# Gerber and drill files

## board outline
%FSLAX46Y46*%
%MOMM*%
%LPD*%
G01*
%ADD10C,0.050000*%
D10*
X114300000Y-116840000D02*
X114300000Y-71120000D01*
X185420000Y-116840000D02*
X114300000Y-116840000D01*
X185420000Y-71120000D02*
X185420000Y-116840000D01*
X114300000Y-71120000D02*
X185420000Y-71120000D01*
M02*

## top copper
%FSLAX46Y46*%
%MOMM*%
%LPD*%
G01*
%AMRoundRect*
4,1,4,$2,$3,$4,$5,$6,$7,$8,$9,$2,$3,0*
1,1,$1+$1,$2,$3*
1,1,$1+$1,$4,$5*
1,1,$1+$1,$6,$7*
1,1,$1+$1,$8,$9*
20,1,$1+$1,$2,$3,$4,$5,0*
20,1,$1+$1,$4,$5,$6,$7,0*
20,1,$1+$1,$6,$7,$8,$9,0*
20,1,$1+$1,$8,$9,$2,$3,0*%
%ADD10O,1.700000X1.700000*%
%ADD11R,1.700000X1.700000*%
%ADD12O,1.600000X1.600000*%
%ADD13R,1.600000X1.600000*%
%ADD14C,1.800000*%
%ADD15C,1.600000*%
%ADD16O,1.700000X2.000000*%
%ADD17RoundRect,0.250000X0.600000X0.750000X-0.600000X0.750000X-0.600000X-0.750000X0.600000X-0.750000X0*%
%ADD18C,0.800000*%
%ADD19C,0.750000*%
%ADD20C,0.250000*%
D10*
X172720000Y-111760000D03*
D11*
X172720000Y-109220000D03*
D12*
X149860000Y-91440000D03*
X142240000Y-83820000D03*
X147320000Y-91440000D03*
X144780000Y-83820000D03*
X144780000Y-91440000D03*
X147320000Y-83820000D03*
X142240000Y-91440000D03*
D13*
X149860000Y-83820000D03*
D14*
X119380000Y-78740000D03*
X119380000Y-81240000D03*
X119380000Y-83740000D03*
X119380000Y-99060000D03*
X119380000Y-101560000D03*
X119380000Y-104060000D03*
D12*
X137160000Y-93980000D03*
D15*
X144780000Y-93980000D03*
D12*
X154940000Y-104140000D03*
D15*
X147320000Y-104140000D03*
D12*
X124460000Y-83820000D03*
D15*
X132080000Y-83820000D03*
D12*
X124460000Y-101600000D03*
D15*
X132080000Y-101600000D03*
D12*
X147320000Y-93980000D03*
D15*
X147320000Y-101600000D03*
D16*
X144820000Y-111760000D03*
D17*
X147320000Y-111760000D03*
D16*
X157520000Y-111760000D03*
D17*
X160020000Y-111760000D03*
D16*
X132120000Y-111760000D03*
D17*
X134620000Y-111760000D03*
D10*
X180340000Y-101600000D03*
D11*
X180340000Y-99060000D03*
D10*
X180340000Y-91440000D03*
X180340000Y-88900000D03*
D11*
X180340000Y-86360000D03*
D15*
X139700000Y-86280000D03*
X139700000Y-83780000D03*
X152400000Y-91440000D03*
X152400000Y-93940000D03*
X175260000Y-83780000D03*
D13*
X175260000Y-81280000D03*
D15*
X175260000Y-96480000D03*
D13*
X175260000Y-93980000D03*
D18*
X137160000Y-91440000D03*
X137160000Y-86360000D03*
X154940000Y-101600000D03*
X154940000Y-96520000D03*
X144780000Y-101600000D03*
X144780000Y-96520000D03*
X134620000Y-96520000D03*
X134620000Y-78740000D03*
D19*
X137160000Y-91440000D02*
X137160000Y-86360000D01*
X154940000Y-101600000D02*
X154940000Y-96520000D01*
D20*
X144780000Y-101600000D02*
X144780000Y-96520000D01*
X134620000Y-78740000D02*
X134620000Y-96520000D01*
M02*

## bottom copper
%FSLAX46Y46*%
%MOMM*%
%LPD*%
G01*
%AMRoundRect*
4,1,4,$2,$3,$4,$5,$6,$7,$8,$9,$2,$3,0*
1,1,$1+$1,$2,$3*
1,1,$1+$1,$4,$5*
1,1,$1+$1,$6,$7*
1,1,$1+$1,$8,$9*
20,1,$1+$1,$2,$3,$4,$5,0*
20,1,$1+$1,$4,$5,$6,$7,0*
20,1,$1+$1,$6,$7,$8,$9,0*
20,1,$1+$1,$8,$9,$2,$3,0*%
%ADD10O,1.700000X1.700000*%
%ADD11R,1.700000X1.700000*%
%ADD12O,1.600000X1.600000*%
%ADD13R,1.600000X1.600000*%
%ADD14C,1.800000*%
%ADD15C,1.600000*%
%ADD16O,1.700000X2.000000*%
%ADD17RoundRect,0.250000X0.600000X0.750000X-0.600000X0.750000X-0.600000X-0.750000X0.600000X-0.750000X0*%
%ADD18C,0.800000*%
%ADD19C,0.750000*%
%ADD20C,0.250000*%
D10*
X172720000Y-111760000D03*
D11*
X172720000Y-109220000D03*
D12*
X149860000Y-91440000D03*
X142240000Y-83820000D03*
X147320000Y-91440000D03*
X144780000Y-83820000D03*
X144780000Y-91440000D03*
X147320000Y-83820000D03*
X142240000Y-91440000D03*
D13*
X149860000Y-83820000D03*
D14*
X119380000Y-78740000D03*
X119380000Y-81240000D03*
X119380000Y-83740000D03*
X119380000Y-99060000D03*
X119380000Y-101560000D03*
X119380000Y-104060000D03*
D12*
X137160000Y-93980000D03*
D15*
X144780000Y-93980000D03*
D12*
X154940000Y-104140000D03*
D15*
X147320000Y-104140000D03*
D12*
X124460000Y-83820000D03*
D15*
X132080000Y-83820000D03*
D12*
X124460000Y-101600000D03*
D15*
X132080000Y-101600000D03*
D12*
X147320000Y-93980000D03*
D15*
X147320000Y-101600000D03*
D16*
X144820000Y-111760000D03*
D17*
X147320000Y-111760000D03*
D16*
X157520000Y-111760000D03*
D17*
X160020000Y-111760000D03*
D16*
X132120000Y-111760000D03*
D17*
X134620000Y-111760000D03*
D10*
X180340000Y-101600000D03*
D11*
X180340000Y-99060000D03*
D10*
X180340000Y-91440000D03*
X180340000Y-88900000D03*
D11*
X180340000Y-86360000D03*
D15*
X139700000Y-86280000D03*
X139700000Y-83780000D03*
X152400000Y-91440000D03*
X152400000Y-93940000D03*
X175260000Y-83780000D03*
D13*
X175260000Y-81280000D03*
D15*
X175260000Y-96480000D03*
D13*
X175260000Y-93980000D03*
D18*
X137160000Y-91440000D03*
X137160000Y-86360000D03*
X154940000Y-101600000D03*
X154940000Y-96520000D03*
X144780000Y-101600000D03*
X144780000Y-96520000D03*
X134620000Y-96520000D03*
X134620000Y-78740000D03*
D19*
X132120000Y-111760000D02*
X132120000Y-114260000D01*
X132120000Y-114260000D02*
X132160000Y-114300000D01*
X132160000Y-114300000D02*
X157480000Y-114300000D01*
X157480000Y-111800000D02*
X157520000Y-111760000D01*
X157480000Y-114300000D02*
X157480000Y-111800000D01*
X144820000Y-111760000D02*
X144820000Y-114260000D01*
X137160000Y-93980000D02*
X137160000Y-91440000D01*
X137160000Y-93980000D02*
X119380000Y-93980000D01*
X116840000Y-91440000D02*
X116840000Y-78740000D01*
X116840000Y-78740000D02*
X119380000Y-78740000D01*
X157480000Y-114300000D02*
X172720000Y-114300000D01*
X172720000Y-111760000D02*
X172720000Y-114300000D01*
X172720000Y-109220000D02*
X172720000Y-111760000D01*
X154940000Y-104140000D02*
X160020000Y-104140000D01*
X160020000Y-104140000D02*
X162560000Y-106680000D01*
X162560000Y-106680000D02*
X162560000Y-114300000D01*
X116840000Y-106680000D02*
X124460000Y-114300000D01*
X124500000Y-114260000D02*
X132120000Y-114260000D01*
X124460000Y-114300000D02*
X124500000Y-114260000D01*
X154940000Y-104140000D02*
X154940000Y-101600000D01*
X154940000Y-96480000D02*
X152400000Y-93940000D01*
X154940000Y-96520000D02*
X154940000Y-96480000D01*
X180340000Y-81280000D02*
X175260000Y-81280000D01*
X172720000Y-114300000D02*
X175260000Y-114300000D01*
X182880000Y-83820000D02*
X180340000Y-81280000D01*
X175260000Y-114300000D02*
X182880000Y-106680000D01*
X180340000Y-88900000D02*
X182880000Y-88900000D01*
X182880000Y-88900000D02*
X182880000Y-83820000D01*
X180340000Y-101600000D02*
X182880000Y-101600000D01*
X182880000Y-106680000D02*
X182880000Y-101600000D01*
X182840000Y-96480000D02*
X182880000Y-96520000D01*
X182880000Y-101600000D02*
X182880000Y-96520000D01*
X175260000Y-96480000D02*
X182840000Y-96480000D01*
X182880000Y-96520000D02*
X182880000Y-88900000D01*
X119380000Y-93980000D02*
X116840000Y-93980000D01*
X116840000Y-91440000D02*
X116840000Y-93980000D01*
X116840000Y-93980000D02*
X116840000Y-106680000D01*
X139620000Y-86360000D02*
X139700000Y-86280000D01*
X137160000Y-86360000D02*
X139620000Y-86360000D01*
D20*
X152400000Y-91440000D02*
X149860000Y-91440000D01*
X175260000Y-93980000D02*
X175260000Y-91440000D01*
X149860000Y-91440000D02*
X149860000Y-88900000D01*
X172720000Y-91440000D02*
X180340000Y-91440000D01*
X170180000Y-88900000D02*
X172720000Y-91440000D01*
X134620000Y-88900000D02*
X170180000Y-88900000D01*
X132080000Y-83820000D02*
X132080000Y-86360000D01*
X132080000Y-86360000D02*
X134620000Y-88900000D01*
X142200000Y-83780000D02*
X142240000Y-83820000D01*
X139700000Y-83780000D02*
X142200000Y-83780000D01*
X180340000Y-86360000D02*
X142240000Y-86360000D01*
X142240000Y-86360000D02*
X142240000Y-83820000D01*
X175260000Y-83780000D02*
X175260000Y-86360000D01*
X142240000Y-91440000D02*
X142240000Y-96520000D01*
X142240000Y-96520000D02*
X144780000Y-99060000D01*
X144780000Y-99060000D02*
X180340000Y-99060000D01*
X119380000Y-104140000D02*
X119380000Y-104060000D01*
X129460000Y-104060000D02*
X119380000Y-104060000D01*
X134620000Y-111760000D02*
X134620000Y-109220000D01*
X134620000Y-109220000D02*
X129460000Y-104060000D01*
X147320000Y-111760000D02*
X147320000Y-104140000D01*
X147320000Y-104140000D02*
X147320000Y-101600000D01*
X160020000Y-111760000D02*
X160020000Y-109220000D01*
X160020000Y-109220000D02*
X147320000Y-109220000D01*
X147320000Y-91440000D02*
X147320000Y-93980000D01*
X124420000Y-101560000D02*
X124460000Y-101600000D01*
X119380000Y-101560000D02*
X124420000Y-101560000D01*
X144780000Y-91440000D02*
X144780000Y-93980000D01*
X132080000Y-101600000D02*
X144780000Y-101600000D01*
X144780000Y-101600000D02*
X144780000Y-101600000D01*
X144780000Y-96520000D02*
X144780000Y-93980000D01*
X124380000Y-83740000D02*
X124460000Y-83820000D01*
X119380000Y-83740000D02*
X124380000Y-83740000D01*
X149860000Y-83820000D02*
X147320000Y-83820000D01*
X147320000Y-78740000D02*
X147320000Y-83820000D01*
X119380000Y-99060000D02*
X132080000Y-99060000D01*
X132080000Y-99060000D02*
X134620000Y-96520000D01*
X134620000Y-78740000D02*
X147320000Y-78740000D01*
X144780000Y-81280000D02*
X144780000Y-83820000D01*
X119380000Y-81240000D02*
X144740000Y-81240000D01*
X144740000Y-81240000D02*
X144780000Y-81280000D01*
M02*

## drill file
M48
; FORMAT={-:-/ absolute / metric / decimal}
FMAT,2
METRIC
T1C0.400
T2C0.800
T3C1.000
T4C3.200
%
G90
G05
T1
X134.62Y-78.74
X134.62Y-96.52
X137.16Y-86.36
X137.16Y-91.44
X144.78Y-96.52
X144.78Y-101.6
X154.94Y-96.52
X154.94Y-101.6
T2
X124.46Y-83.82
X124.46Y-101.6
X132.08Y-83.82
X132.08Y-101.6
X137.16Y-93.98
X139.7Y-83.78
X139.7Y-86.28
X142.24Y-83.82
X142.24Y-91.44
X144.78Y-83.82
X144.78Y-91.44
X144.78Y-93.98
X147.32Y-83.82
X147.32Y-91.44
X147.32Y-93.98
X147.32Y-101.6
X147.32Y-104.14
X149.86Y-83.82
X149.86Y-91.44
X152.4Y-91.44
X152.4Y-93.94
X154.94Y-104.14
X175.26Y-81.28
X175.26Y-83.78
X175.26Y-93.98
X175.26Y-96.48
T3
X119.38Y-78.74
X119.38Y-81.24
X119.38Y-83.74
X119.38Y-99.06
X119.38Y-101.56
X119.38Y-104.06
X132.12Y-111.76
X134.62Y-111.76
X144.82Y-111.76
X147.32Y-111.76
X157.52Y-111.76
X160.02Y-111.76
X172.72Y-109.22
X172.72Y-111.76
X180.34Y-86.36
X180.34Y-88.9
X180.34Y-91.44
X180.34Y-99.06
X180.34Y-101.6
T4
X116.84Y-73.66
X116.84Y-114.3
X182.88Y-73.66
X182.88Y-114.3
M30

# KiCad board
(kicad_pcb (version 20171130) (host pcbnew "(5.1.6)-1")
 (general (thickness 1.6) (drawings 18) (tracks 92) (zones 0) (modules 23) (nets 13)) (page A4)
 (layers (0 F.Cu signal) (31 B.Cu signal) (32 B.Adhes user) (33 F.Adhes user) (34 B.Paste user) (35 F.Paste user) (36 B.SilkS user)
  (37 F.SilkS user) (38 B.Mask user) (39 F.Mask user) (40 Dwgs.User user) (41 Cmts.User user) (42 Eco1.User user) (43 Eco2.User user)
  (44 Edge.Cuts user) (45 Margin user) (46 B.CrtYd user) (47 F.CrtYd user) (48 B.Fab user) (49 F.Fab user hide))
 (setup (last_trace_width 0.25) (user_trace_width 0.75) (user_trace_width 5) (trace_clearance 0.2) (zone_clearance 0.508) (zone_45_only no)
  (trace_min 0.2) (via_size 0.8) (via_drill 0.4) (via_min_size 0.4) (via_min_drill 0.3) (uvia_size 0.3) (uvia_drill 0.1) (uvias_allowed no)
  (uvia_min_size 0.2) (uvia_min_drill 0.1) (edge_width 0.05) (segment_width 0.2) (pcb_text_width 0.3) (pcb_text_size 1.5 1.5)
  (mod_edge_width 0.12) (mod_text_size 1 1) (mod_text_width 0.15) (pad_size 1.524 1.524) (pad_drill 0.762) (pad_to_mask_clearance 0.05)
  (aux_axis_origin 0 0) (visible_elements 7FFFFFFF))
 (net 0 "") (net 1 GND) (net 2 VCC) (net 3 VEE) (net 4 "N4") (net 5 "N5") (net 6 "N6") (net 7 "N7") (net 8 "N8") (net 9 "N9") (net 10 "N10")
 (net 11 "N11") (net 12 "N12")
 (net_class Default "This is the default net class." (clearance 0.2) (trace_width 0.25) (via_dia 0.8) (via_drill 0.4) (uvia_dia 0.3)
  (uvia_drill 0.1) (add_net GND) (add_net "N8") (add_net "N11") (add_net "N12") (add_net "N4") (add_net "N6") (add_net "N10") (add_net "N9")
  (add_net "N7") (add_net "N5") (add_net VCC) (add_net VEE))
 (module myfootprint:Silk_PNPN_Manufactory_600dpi (layer F.Cu) (at 163.195 81.28)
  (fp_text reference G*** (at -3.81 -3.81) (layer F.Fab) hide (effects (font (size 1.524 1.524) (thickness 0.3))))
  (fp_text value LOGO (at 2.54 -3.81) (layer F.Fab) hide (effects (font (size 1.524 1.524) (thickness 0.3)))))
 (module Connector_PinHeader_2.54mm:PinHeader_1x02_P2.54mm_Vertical (layer F.Cu) (at 172.72 109.22)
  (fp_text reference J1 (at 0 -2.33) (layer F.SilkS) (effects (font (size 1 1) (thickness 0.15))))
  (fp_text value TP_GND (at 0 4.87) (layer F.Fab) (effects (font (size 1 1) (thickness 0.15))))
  (pad 2 thru_hole oval (at 0 2.54) (size 1.7 1.7) (drill 1) (layers *.Cu *.Mask) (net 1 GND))
  (pad 1 thru_hole rect (at 0 0) (size 1.7 1.7) (drill 1) (layers *.Cu *.Mask) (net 1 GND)))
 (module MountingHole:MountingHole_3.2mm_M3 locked (layer F.Cu) (at 182.88 114.3)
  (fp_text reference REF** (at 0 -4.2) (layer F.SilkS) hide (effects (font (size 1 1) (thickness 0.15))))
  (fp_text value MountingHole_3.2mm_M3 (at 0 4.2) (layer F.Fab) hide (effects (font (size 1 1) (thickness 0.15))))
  (pad 1 np_thru_hole circle (at 0 0) (size 3.2 3.2) (drill 3.2) (layers *.Cu *.Mask)))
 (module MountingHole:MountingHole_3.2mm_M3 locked (layer F.Cu) (at 182.88 73.66)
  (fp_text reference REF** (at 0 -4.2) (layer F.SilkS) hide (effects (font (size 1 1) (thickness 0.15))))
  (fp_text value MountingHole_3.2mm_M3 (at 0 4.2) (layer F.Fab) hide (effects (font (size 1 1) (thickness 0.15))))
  (pad 1 np_thru_hole circle (at 0 0) (size 3.2 3.2) (drill 3.2) (layers *.Cu *.Mask)))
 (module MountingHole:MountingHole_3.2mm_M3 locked (layer F.Cu) (at 116.84 114.3)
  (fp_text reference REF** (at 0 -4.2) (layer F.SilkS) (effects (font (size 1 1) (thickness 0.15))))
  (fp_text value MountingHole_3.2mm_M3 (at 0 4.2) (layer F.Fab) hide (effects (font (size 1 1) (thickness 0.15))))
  (pad 1 np_thru_hole circle (at 0 0) (size 3.2 3.2) (drill 3.2) (layers *.Cu *.Mask)))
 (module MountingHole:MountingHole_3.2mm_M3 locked (layer F.Cu) (at 116.84 73.66)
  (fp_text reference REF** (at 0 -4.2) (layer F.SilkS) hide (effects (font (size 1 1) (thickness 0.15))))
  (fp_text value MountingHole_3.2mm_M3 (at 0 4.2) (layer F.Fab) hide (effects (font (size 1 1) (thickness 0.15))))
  (pad 1 np_thru_hole circle (at 0 0) (size 3.2 3.2) (drill 3.2) (layers *.Cu *.Mask)))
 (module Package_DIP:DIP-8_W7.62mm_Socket (layer F.Cu) (at 149.86 83.82 270)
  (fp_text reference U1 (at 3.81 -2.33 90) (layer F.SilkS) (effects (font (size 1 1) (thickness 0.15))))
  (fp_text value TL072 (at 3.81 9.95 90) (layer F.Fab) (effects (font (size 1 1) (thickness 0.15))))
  (pad 8 thru_hole oval (at 7.62 0 270) (size 1.6 1.6) (drill 0.8) (layers *.Cu *.Mask) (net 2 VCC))
  (pad 4 thru_hole oval (at 0 7.62 270) (size 1.6 1.6) (drill 0.8) (layers *.Cu *.Mask) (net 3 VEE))
  (pad 7 thru_hole oval (at 7.62 2.54 270) (size 1.6 1.6) (drill 0.8) (layers *.Cu *.Mask) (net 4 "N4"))
  (pad 3 thru_hole oval (at 0 5.08 270) (size 1.6 1.6) (drill 0.8) (layers *.Cu *.Mask) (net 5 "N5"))
  (pad 6 thru_hole oval (at 7.62 5.08 270) (size 1.6 1.6) (drill 0.8) (layers *.Cu *.Mask) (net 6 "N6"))
  (pad 2 thru_hole oval (at 0 2.54 270) (size 1.6 1.6) (drill 0.8) (layers *.Cu *.Mask) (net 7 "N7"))
  (pad 5 thru_hole oval (at 7.62 7.62 270) (size 1.6 1.6) (drill 0.8) (layers *.Cu *.Mask) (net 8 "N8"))
  (pad 1 thru_hole rect (at 0 0 270) (size 1.6 1.6) (drill 0.8) (layers *.Cu *.Mask) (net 7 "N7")))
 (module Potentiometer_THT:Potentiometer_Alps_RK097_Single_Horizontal (layer F.Cu) (at 119.38 78.74 180)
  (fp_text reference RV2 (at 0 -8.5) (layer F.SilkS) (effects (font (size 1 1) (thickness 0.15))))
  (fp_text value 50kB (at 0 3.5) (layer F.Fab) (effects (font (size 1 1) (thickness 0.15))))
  (pad 1 thru_hole circle (at 0 0 180) (size 1.8 1.8) (drill 1) (layers *.Cu *.Mask) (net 1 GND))
  (pad 2 thru_hole circle (at 0 -2.5 180) (size 1.8 1.8) (drill 1) (layers *.Cu *.Mask) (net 5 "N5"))
  (pad 3 thru_hole circle (at 0 -5 180) (size 1.8 1.8) (drill 1) (layers *.Cu *.Mask) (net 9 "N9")))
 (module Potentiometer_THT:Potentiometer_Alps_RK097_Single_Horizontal (layer F.Cu) (at 119.38 99.06 180)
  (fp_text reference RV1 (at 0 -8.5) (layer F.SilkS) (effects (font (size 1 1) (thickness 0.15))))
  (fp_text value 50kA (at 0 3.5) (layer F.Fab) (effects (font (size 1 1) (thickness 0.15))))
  (pad 1 thru_hole circle (at 0 0 180) (size 1.8 1.8) (drill 1) (layers *.Cu *.Mask) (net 7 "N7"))
  (pad 2 thru_hole circle (at 0 -2.5 180) (size 1.8 1.8) (drill 1) (layers *.Cu *.Mask) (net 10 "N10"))
  (pad 3 thru_hole circle (at 0 -5 180) (size 1.8 1.8) (drill 1) (layers *.Cu *.Mask) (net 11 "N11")))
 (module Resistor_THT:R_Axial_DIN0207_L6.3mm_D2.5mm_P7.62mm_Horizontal (layer F.Cu) (at 144.78 93.98 180)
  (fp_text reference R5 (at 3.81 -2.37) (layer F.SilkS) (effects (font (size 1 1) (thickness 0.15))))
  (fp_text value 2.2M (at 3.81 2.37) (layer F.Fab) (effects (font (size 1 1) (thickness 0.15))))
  (pad 2 thru_hole oval (at 7.62 0 180) (size 1.6 1.6) (drill 0.8) (layers *.Cu *.Mask) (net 1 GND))
  (pad 1 thru_hole circle (at 0 0 180) (size 1.6 1.6) (drill 0.8) (layers *.Cu *.Mask) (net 6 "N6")))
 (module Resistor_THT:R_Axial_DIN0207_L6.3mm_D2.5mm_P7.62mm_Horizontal (layer F.Cu) (at 147.32 104.14)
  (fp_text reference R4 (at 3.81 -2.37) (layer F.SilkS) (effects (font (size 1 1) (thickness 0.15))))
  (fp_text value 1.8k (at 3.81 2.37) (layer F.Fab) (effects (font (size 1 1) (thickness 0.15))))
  (pad 2 thru_hole oval (at 7.62 0) (size 1.6 1.6) (drill 0.8) (layers *.Cu *.Mask) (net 1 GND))
  (pad 1 thru_hole circle (at 0 0) (size 1.6 1.6) (drill 0.8) (layers *.Cu *.Mask) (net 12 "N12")))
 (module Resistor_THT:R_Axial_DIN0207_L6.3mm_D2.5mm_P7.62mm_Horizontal (layer F.Cu) (at 132.08 83.82 180)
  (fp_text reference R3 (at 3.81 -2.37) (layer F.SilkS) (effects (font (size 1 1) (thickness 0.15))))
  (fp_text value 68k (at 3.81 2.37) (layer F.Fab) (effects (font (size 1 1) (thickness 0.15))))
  (pad 2 thru_hole oval (at 7.62 0 180) (size 1.6 1.6) (drill 0.8) (layers *.Cu *.Mask) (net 9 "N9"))
  (pad 1 thru_hole circle (at 0 0 180) (size 1.6 1.6) (drill 0.8) (layers *.Cu *.Mask) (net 2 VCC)))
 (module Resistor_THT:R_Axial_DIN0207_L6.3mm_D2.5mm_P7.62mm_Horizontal (layer F.Cu) (at 132.08 101.6 180)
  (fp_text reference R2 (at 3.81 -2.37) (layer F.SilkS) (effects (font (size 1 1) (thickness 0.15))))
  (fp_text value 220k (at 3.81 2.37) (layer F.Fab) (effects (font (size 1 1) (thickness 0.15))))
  (pad 2 thru_hole oval (at 7.62 0 180) (size 1.6 1.6) (drill 0.8) (layers *.Cu *.Mask) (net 10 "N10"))
  (pad 1 thru_hole circle (at 0 0 180) (size 1.6 1.6) (drill 0.8) (layers *.Cu *.Mask) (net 6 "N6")))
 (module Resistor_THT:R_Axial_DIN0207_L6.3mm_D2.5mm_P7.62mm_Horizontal (layer F.Cu) (at 147.32 101.6 90)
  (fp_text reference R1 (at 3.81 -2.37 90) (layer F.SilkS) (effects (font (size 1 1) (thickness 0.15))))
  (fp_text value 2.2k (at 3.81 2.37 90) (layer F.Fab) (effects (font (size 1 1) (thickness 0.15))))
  (pad 2 thru_hole oval (at 7.62 0 90) (size 1.6 1.6) (drill 0.8) (layers *.Cu *.Mask) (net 4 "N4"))
  (pad 1 thru_hole circle (at 0 0 90) (size 1.6 1.6) (drill 0.8) (layers *.Cu *.Mask) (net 12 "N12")))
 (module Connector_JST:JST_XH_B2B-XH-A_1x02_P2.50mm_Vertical (layer F.Cu) (at 147.32 111.76 180)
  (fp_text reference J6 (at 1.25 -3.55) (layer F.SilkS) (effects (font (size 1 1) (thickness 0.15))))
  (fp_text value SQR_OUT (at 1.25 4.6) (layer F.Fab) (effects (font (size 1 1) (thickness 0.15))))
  (pad 2 thru_hole oval (at 2.5 0 180) (size 1.7 2) (drill 1) (layers *.Cu *.Mask) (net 1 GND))
  (pad 1 thru_hole roundrect (at 0 0 180) (size 1.7 2) (drill 1) (layers *.Cu *.Mask) (roundrect_rratio 0.147059) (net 12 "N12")))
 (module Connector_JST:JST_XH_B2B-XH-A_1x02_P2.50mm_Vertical (layer F.Cu) (at 160.02 111.76 180)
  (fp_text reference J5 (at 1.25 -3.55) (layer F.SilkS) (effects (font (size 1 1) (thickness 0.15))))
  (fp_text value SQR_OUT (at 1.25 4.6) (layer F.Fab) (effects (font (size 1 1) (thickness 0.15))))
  (pad 2 thru_hole oval (at 2.5 0 180) (size 1.7 2) (drill 1) (layers *.Cu *.Mask) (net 1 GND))
  (pad 1 thru_hole roundrect (at 0 0 180) (size 1.7 2) (drill 1) (layers *.Cu *.Mask) (roundrect_rratio 0.147059) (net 12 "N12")))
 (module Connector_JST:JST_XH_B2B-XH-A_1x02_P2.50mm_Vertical (layer F.Cu) (at 134.62 111.76 180)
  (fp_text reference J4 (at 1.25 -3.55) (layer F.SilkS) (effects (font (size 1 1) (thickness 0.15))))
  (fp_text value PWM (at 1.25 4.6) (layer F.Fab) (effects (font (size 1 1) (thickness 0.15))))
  (pad 2 thru_hole oval (at 2.5 0 180) (size 1.7 2) (drill 1) (layers *.Cu *.Mask) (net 1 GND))
  (pad 1 thru_hole roundrect (at 0 0 180) (size 1.7 2) (drill 1) (layers *.Cu *.Mask) (roundrect_rratio 0.147059) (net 11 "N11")))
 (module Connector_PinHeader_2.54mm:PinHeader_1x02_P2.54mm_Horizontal (layer F.Cu) (at 180.34 99.06)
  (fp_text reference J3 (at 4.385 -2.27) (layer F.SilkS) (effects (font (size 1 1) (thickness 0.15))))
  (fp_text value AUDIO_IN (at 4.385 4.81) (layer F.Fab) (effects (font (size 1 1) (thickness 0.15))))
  (pad 2 thru_hole oval (at 0 2.54) (size 1.7 1.7) (drill 1) (layers *.Cu *.Mask) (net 1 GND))
  (pad 1 thru_hole rect (at 0 0) (size 1.7 1.7) (drill 1) (layers *.Cu *.Mask) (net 8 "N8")))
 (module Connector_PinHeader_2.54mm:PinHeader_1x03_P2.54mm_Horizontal (layer F.Cu) (at 180.34 86.36)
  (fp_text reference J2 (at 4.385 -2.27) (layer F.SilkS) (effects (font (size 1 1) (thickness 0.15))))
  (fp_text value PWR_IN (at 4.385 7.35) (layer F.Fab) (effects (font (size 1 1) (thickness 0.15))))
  (pad 3 thru_hole oval (at 0 5.08) (size 1.7 1.7) (drill 1) (layers *.Cu *.Mask) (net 2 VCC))
  (pad 2 thru_hole oval (at 0 2.54) (size 1.7 1.7) (drill 1) (layers *.Cu *.Mask) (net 1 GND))
  (pad 1 thru_hole rect (at 0 0) (size 1.7 1.7) (drill 1) (layers *.Cu *.Mask) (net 3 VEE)))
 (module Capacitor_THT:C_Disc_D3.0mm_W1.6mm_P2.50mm (layer F.Cu) (at 139.7 83.78 270)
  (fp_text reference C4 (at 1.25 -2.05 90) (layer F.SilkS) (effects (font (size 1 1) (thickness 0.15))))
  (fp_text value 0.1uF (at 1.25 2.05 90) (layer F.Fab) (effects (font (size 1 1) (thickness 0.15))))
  (pad 2 thru_hole circle (at 2.5 0 270) (size 1.6 1.6) (drill 0.8) (layers *.Cu *.Mask) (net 1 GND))
  (pad 1 thru_hole circle (at 0 0 270) (size 1.6 1.6) (drill 0.8) (layers *.Cu *.Mask) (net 3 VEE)))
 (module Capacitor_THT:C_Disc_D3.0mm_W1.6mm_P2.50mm (layer F.Cu) (at 152.4 93.94 90)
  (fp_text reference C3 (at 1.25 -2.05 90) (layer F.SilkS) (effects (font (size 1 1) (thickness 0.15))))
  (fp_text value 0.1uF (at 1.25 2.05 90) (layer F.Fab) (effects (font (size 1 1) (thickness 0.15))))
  (pad 2 thru_hole circle (at 2.5 0 90) (size 1.6 1.6) (drill 0.8) (layers *.Cu *.Mask) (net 2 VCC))
  (pad 1 thru_hole circle (at 0 0 90) (size 1.6 1.6) (drill 0.8) (layers *.Cu *.Mask) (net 1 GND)))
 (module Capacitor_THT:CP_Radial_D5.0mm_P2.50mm (layer F.Cu) (at 175.26 81.28 270)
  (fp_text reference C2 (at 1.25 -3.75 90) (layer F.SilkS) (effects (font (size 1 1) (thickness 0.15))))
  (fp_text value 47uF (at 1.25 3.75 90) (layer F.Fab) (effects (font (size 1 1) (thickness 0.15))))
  (pad 2 thru_hole circle (at 2.5 0 270) (size 1.6 1.6) (drill 0.8) (layers *.Cu *.Mask) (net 3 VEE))
  (pad 1 thru_hole rect (at 0 0 270) (size 1.6 1.6) (drill 0.8) (layers *.Cu *.Mask) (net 1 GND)))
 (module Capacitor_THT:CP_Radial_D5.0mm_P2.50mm (layer F.Cu) (at 175.26 93.98 270)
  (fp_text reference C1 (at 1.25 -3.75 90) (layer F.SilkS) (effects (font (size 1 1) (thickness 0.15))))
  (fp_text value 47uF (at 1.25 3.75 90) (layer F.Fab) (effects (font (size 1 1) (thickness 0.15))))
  (pad 2 thru_hole circle (at 2.5 0 270) (size 1.6 1.6) (drill 0.8) (layers *.Cu *.Mask) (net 1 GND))
  (pad 1 thru_hole rect (at 0 0 270) (size 1.6 1.6) (drill 0.8) (layers *.Cu *.Mask) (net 2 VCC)))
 (gr_line (start 114.3 116.84) (end 114.3 71.12) (layer Edge.Cuts) (width 0.05))
 (gr_line (start 185.42 116.84) (end 114.3 116.84) (layer Edge.Cuts) (width 0.05))
 (gr_line (start 185.42 71.12) (end 185.42 116.84) (layer Edge.Cuts) (width 0.05))
 (gr_line (start 114.3 71.12) (end 185.42 71.12) (layer Edge.Cuts) (width 0.05))
 (segment (start 132.12 111.76) (end 132.12 114.26) (width 0.75) (layer B.Cu) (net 1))
 (segment (start 132.12 114.26) (end 132.16 114.3) (width 0.75) (layer B.Cu) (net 1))
 (segment (start 132.16 114.3) (end 157.48 114.3) (width 0.75) (layer B.Cu) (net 1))
 (segment (start 157.48 111.8) (end 157.52 111.76) (width 0.75) (layer B.Cu) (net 1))
 (segment (start 157.48 114.3) (end 157.48 111.8) (width 0.75) (layer B.Cu) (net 1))
 (segment (start 144.82 111.76) (end 144.82 114.26) (width 0.75) (layer B.Cu) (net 1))
 (segment (start 137.16 93.98) (end 137.16 91.44) (width 0.75) (layer B.Cu) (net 1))
 (via (at 137.16 91.44) (size 0.8) (drill 0.4) (layers F.Cu B.Cu) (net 1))
 (segment (start 137.16 91.44) (end 137.16 86.36) (width 0.75) (layer F.Cu) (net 1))
 (via (at 137.16 86.36) (size 0.8) (drill 0.4) (layers F.Cu B.Cu) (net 1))
 (segment (start 137.16 93.98) (end 119.38 93.98) (width 0.75) (layer B.Cu) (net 1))
 (segment (start 116.84 91.44) (end 116.84 78.74) (width 0.75) (layer B.Cu) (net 1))
 (segment (start 116.84 78.74) (end 119.38 78.74) (width 0.75) (layer B.Cu) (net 1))
 (segment (start 157.48 114.3) (end 172.72 114.3) (width 0.75) (layer B.Cu) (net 1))
 (segment (start 172.72 111.76) (end 172.72 114.3) (width 0.75) (layer B.Cu) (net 1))
 (segment (start 172.72 109.22) (end 172.72 111.76) (width 0.75) (layer B.Cu) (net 1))
 (segment (start 154.94 104.14) (end 160.02 104.14) (width 0.75) (layer B.Cu) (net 1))
 (segment (start 160.02 104.14) (end 162.56 106.68) (width 0.75) (layer B.Cu) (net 1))
 (segment (start 162.56 106.68) (end 162.56 114.3) (width 0.75) (layer B.Cu) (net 1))
 (segment (start 116.84 106.68) (end 124.46 114.3) (width 0.75) (layer B.Cu) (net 1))
 (segment (start 124.5 114.26) (end 132.12 114.26) (width 0.75) (layer B.Cu) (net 1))
 (segment (start 124.46 114.3) (end 124.5 114.26) (width 0.75) (layer B.Cu) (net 1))
 (segment (start 154.94 104.14) (end 154.94 101.6) (width 0.75) (layer B.Cu) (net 1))
 (via (at 154.94 101.6) (size 0.8) (drill 0.4) (layers F.Cu B.Cu) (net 1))
 (segment (start 154.94 101.6) (end 154.94 96.52) (width 0.75) (layer F.Cu) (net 1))
 (via (at 154.94 96.52) (size 0.8) (drill 0.4) (layers F.Cu B.Cu) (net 1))
 (segment (start 154.94 96.48) (end 152.4 93.94) (width 0.75) (layer B.Cu) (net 1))
 (segment (start 154.94 96.52) (end 154.94 96.48) (width 0.75) (layer B.Cu) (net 1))
 (segment (start 180.34 81.28) (end 175.26 81.28) (width 0.75) (layer B.Cu) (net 1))
 (segment (start 172.72 114.3) (end 175.26 114.3) (width 0.75) (layer B.Cu) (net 1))
 (segment (start 182.88 83.82) (end 180.34 81.28) (width 0.75) (layer B.Cu) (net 1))
 (segment (start 175.26 114.3) (end 182.88 106.68) (width 0.75) (layer B.Cu) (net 1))
 (segment (start 180.34 88.9) (end 182.88 88.9) (width 0.75) (layer B.Cu) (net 1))
 (segment (start 182.88 88.9) (end 182.88 83.82) (width 0.75) (layer B.Cu) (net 1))
 (segment (start 180.34 101.6) (end 182.88 101.6) (width 0.75) (layer B.Cu) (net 1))
 (segment (start 182.88 106.68) (end 182.88 101.6) (width 0.75) (layer B.Cu) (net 1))
 (segment (start 182.84 96.48) (end 182.88 96.52) (width 0.75) (layer B.Cu) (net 1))
 (segment (start 182.88 101.6) (end 182.88 96.52) (width 0.75) (layer B.Cu) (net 1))
 (segment (start 175.26 96.48) (end 182.84 96.48) (width 0.75) (layer B.Cu) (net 1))
 (segment (start 182.88 96.52) (end 182.88 88.9) (width 0.75) (layer B.Cu) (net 1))
 (segment (start 119.38 93.98) (end 116.84 93.98) (width 0.75) (layer B.Cu) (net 1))
 (segment (start 116.84 91.44) (end 116.84 93.98) (width 0.75) (layer B.Cu) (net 1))
 (segment (start 116.84 93.98) (end 116.84 106.68) (width 0.75) (layer B.Cu) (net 1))
 (segment (start 139.62 86.36) (end 139.7 86.28) (width 0.75) (layer B.Cu) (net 1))
 (segment (start 137.16 86.36) (end 139.62 86.36) (width 0.75) (layer B.Cu) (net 1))
 (segment (start 152.4 91.44) (end 149.86 91.44) (width 0.25) (layer B.Cu) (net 2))
 (segment (start 175.26 93.98) (end 175.26 91.44) (width 0.25) (layer B.Cu) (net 2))
 (segment (start 149.86 91.44) (end 149.86 88.9) (width 0.25) (layer B.Cu) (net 2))
 (segment (start 172.72 91.44) (end 180.34 91.44) (width 0.25) (layer B.Cu) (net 2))
 (segment (start 170.18 88.9) (end 172.72 91.44) (width 0.25) (layer B.Cu) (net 2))
 (segment (start 134.62 88.9) (end 170.18 88.9) (width 0.25) (layer B.Cu) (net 2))
 (segment (start 132.08 83.82) (end 132.08 86.36) (width 0.25) (layer B.Cu) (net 2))
 (segment (start 132.08 86.36) (end 134.62 88.9) (width 0.25) (layer B.Cu) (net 2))
 (segment (start 142.2 83.78) (end 142.24 83.82) (width 0.25) (layer B.Cu) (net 3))
 (segment (start 139.7 83.78) (end 142.2 83.78) (width 0.25) (layer B.Cu) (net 3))
 (segment (start 180.34 86.36) (end 142.24 86.36) (width 0.25) (layer B.Cu) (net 3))
 (segment (start 142.24 86.36) (end 142.24 83.82) (width 0.25) (layer B.Cu) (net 3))
 (segment (start 175.26 83.78) (end 175.26 86.36) (width 0.25) (layer B.Cu) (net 3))
 (segment (start 142.24 91.44) (end 142.24 96.52) (width 0.25) (layer B.Cu) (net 8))
 (segment (start 142.24 96.52) (end 144.78 99.06) (width 0.25) (layer B.Cu) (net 8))
 (segment (start 144.78 99.06) (end 180.34 99.06) (width 0.25) (layer B.Cu) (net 8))
 (segment (start 119.38 104.14) (end 119.38 104.06) (width 0.25) (layer B.Cu) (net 11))
 (segment (start 129.46 104.06) (end 119.38 104.06) (width 0.25) (layer B.Cu) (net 11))
 (segment (start 134.62 111.76) (end 134.62 109.22) (width 0.25) (layer B.Cu) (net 11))
 (segment (start 134.62 109.22) (end 129.46 104.06) (width 0.25) (layer B.Cu) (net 11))
 (segment (start 147.32 111.76) (end 147.32 104.14) (width 0.25) (layer B.Cu) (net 12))
 (segment (start 147.32 104.14) (end 147.32 101.6) (width 0.25) (layer B.Cu) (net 12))
 (segment (start 160.02 111.76) (end 160.02 109.22) (width 0.25) (layer B.Cu) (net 12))
 (segment (start 160.02 109.22) (end 147.32 109.22) (width 0.25) (layer B.Cu) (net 12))
 (segment (start 147.32 91.44) (end 147.32 93.98) (width 0.25) (layer B.Cu) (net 4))
 (segment (start 124.42 101.56) (end 124.46 101.6) (width 0.25) (layer B.Cu) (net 10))
 (segment (start 119.38 101.56) (end 124.42 101.56) (width 0.25) (layer B.Cu) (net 10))
 (segment (start 144.78 91.44) (end 144.78 93.98) (width 0.25) (layer B.Cu) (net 6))
 (segment (start 132.08 101.6) (end 144.78 101.6) (width 0.25) (layer B.Cu) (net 6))
 (segment (start 144.78 101.6) (end 144.78 101.6) (width 0.25) (layer B.Cu) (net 6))
 (via (at 144.78 101.6) (size 0.8) (drill 0.4) (layers F.Cu B.Cu) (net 6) (status 1000000))
 (segment (start 144.78 101.6) (end 144.78 96.52) (width 0.25) (layer F.Cu) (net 6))
 (via (at 144.78 96.52) (size 0.8) (drill 0.4) (layers F.Cu B.Cu) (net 6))
 (segment (start 144.78 96.52) (end 144.78 93.98) (width 0.25) (layer B.Cu) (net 6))
 (segment (start 124.38 83.74) (end 124.46 83.82) (width 0.25) (layer B.Cu) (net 9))
 (segment (start 119.38 83.74) (end 124.38 83.74) (width 0.25) (layer B.Cu) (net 9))
 (segment (start 149.86 83.82) (end 147.32 83.82) (width 0.25) (layer B.Cu) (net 7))
 (segment (start 147.32 78.74) (end 147.32 83.82) (width 0.25) (layer B.Cu) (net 7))
 (via (at 134.62 96.52) (size 0.8) (drill 0.4) (layers F.Cu B.Cu) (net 7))
 (segment (start 119.38 99.06) (end 132.08 99.06) (width 0.25) (layer B.Cu) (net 7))
 (segment (start 132.08 99.06) (end 134.62 96.52) (width 0.25) (layer B.Cu) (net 7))
 (segment (start 134.62 78.74) (end 134.62 96.52) (width 0.25) (layer F.Cu) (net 7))
 (via (at 134.62 78.74) (size 0.8) (drill 0.4) (layers F.Cu B.Cu) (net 7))
 (segment (start 134.62 78.74) (end 147.32 78.74) (width 0.25) (layer B.Cu) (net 7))
 (segment (start 144.78 81.28) (end 144.78 83.82) (width 0.25) (layer B.Cu) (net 5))
 (segment (start 119.38 81.24) (end 144.74 81.24) (width 0.25) (layer B.Cu) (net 5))
 (segment (start 144.74 81.24) (end 144.78 81.28) (width 0.25) (layer B.Cu) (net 5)))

